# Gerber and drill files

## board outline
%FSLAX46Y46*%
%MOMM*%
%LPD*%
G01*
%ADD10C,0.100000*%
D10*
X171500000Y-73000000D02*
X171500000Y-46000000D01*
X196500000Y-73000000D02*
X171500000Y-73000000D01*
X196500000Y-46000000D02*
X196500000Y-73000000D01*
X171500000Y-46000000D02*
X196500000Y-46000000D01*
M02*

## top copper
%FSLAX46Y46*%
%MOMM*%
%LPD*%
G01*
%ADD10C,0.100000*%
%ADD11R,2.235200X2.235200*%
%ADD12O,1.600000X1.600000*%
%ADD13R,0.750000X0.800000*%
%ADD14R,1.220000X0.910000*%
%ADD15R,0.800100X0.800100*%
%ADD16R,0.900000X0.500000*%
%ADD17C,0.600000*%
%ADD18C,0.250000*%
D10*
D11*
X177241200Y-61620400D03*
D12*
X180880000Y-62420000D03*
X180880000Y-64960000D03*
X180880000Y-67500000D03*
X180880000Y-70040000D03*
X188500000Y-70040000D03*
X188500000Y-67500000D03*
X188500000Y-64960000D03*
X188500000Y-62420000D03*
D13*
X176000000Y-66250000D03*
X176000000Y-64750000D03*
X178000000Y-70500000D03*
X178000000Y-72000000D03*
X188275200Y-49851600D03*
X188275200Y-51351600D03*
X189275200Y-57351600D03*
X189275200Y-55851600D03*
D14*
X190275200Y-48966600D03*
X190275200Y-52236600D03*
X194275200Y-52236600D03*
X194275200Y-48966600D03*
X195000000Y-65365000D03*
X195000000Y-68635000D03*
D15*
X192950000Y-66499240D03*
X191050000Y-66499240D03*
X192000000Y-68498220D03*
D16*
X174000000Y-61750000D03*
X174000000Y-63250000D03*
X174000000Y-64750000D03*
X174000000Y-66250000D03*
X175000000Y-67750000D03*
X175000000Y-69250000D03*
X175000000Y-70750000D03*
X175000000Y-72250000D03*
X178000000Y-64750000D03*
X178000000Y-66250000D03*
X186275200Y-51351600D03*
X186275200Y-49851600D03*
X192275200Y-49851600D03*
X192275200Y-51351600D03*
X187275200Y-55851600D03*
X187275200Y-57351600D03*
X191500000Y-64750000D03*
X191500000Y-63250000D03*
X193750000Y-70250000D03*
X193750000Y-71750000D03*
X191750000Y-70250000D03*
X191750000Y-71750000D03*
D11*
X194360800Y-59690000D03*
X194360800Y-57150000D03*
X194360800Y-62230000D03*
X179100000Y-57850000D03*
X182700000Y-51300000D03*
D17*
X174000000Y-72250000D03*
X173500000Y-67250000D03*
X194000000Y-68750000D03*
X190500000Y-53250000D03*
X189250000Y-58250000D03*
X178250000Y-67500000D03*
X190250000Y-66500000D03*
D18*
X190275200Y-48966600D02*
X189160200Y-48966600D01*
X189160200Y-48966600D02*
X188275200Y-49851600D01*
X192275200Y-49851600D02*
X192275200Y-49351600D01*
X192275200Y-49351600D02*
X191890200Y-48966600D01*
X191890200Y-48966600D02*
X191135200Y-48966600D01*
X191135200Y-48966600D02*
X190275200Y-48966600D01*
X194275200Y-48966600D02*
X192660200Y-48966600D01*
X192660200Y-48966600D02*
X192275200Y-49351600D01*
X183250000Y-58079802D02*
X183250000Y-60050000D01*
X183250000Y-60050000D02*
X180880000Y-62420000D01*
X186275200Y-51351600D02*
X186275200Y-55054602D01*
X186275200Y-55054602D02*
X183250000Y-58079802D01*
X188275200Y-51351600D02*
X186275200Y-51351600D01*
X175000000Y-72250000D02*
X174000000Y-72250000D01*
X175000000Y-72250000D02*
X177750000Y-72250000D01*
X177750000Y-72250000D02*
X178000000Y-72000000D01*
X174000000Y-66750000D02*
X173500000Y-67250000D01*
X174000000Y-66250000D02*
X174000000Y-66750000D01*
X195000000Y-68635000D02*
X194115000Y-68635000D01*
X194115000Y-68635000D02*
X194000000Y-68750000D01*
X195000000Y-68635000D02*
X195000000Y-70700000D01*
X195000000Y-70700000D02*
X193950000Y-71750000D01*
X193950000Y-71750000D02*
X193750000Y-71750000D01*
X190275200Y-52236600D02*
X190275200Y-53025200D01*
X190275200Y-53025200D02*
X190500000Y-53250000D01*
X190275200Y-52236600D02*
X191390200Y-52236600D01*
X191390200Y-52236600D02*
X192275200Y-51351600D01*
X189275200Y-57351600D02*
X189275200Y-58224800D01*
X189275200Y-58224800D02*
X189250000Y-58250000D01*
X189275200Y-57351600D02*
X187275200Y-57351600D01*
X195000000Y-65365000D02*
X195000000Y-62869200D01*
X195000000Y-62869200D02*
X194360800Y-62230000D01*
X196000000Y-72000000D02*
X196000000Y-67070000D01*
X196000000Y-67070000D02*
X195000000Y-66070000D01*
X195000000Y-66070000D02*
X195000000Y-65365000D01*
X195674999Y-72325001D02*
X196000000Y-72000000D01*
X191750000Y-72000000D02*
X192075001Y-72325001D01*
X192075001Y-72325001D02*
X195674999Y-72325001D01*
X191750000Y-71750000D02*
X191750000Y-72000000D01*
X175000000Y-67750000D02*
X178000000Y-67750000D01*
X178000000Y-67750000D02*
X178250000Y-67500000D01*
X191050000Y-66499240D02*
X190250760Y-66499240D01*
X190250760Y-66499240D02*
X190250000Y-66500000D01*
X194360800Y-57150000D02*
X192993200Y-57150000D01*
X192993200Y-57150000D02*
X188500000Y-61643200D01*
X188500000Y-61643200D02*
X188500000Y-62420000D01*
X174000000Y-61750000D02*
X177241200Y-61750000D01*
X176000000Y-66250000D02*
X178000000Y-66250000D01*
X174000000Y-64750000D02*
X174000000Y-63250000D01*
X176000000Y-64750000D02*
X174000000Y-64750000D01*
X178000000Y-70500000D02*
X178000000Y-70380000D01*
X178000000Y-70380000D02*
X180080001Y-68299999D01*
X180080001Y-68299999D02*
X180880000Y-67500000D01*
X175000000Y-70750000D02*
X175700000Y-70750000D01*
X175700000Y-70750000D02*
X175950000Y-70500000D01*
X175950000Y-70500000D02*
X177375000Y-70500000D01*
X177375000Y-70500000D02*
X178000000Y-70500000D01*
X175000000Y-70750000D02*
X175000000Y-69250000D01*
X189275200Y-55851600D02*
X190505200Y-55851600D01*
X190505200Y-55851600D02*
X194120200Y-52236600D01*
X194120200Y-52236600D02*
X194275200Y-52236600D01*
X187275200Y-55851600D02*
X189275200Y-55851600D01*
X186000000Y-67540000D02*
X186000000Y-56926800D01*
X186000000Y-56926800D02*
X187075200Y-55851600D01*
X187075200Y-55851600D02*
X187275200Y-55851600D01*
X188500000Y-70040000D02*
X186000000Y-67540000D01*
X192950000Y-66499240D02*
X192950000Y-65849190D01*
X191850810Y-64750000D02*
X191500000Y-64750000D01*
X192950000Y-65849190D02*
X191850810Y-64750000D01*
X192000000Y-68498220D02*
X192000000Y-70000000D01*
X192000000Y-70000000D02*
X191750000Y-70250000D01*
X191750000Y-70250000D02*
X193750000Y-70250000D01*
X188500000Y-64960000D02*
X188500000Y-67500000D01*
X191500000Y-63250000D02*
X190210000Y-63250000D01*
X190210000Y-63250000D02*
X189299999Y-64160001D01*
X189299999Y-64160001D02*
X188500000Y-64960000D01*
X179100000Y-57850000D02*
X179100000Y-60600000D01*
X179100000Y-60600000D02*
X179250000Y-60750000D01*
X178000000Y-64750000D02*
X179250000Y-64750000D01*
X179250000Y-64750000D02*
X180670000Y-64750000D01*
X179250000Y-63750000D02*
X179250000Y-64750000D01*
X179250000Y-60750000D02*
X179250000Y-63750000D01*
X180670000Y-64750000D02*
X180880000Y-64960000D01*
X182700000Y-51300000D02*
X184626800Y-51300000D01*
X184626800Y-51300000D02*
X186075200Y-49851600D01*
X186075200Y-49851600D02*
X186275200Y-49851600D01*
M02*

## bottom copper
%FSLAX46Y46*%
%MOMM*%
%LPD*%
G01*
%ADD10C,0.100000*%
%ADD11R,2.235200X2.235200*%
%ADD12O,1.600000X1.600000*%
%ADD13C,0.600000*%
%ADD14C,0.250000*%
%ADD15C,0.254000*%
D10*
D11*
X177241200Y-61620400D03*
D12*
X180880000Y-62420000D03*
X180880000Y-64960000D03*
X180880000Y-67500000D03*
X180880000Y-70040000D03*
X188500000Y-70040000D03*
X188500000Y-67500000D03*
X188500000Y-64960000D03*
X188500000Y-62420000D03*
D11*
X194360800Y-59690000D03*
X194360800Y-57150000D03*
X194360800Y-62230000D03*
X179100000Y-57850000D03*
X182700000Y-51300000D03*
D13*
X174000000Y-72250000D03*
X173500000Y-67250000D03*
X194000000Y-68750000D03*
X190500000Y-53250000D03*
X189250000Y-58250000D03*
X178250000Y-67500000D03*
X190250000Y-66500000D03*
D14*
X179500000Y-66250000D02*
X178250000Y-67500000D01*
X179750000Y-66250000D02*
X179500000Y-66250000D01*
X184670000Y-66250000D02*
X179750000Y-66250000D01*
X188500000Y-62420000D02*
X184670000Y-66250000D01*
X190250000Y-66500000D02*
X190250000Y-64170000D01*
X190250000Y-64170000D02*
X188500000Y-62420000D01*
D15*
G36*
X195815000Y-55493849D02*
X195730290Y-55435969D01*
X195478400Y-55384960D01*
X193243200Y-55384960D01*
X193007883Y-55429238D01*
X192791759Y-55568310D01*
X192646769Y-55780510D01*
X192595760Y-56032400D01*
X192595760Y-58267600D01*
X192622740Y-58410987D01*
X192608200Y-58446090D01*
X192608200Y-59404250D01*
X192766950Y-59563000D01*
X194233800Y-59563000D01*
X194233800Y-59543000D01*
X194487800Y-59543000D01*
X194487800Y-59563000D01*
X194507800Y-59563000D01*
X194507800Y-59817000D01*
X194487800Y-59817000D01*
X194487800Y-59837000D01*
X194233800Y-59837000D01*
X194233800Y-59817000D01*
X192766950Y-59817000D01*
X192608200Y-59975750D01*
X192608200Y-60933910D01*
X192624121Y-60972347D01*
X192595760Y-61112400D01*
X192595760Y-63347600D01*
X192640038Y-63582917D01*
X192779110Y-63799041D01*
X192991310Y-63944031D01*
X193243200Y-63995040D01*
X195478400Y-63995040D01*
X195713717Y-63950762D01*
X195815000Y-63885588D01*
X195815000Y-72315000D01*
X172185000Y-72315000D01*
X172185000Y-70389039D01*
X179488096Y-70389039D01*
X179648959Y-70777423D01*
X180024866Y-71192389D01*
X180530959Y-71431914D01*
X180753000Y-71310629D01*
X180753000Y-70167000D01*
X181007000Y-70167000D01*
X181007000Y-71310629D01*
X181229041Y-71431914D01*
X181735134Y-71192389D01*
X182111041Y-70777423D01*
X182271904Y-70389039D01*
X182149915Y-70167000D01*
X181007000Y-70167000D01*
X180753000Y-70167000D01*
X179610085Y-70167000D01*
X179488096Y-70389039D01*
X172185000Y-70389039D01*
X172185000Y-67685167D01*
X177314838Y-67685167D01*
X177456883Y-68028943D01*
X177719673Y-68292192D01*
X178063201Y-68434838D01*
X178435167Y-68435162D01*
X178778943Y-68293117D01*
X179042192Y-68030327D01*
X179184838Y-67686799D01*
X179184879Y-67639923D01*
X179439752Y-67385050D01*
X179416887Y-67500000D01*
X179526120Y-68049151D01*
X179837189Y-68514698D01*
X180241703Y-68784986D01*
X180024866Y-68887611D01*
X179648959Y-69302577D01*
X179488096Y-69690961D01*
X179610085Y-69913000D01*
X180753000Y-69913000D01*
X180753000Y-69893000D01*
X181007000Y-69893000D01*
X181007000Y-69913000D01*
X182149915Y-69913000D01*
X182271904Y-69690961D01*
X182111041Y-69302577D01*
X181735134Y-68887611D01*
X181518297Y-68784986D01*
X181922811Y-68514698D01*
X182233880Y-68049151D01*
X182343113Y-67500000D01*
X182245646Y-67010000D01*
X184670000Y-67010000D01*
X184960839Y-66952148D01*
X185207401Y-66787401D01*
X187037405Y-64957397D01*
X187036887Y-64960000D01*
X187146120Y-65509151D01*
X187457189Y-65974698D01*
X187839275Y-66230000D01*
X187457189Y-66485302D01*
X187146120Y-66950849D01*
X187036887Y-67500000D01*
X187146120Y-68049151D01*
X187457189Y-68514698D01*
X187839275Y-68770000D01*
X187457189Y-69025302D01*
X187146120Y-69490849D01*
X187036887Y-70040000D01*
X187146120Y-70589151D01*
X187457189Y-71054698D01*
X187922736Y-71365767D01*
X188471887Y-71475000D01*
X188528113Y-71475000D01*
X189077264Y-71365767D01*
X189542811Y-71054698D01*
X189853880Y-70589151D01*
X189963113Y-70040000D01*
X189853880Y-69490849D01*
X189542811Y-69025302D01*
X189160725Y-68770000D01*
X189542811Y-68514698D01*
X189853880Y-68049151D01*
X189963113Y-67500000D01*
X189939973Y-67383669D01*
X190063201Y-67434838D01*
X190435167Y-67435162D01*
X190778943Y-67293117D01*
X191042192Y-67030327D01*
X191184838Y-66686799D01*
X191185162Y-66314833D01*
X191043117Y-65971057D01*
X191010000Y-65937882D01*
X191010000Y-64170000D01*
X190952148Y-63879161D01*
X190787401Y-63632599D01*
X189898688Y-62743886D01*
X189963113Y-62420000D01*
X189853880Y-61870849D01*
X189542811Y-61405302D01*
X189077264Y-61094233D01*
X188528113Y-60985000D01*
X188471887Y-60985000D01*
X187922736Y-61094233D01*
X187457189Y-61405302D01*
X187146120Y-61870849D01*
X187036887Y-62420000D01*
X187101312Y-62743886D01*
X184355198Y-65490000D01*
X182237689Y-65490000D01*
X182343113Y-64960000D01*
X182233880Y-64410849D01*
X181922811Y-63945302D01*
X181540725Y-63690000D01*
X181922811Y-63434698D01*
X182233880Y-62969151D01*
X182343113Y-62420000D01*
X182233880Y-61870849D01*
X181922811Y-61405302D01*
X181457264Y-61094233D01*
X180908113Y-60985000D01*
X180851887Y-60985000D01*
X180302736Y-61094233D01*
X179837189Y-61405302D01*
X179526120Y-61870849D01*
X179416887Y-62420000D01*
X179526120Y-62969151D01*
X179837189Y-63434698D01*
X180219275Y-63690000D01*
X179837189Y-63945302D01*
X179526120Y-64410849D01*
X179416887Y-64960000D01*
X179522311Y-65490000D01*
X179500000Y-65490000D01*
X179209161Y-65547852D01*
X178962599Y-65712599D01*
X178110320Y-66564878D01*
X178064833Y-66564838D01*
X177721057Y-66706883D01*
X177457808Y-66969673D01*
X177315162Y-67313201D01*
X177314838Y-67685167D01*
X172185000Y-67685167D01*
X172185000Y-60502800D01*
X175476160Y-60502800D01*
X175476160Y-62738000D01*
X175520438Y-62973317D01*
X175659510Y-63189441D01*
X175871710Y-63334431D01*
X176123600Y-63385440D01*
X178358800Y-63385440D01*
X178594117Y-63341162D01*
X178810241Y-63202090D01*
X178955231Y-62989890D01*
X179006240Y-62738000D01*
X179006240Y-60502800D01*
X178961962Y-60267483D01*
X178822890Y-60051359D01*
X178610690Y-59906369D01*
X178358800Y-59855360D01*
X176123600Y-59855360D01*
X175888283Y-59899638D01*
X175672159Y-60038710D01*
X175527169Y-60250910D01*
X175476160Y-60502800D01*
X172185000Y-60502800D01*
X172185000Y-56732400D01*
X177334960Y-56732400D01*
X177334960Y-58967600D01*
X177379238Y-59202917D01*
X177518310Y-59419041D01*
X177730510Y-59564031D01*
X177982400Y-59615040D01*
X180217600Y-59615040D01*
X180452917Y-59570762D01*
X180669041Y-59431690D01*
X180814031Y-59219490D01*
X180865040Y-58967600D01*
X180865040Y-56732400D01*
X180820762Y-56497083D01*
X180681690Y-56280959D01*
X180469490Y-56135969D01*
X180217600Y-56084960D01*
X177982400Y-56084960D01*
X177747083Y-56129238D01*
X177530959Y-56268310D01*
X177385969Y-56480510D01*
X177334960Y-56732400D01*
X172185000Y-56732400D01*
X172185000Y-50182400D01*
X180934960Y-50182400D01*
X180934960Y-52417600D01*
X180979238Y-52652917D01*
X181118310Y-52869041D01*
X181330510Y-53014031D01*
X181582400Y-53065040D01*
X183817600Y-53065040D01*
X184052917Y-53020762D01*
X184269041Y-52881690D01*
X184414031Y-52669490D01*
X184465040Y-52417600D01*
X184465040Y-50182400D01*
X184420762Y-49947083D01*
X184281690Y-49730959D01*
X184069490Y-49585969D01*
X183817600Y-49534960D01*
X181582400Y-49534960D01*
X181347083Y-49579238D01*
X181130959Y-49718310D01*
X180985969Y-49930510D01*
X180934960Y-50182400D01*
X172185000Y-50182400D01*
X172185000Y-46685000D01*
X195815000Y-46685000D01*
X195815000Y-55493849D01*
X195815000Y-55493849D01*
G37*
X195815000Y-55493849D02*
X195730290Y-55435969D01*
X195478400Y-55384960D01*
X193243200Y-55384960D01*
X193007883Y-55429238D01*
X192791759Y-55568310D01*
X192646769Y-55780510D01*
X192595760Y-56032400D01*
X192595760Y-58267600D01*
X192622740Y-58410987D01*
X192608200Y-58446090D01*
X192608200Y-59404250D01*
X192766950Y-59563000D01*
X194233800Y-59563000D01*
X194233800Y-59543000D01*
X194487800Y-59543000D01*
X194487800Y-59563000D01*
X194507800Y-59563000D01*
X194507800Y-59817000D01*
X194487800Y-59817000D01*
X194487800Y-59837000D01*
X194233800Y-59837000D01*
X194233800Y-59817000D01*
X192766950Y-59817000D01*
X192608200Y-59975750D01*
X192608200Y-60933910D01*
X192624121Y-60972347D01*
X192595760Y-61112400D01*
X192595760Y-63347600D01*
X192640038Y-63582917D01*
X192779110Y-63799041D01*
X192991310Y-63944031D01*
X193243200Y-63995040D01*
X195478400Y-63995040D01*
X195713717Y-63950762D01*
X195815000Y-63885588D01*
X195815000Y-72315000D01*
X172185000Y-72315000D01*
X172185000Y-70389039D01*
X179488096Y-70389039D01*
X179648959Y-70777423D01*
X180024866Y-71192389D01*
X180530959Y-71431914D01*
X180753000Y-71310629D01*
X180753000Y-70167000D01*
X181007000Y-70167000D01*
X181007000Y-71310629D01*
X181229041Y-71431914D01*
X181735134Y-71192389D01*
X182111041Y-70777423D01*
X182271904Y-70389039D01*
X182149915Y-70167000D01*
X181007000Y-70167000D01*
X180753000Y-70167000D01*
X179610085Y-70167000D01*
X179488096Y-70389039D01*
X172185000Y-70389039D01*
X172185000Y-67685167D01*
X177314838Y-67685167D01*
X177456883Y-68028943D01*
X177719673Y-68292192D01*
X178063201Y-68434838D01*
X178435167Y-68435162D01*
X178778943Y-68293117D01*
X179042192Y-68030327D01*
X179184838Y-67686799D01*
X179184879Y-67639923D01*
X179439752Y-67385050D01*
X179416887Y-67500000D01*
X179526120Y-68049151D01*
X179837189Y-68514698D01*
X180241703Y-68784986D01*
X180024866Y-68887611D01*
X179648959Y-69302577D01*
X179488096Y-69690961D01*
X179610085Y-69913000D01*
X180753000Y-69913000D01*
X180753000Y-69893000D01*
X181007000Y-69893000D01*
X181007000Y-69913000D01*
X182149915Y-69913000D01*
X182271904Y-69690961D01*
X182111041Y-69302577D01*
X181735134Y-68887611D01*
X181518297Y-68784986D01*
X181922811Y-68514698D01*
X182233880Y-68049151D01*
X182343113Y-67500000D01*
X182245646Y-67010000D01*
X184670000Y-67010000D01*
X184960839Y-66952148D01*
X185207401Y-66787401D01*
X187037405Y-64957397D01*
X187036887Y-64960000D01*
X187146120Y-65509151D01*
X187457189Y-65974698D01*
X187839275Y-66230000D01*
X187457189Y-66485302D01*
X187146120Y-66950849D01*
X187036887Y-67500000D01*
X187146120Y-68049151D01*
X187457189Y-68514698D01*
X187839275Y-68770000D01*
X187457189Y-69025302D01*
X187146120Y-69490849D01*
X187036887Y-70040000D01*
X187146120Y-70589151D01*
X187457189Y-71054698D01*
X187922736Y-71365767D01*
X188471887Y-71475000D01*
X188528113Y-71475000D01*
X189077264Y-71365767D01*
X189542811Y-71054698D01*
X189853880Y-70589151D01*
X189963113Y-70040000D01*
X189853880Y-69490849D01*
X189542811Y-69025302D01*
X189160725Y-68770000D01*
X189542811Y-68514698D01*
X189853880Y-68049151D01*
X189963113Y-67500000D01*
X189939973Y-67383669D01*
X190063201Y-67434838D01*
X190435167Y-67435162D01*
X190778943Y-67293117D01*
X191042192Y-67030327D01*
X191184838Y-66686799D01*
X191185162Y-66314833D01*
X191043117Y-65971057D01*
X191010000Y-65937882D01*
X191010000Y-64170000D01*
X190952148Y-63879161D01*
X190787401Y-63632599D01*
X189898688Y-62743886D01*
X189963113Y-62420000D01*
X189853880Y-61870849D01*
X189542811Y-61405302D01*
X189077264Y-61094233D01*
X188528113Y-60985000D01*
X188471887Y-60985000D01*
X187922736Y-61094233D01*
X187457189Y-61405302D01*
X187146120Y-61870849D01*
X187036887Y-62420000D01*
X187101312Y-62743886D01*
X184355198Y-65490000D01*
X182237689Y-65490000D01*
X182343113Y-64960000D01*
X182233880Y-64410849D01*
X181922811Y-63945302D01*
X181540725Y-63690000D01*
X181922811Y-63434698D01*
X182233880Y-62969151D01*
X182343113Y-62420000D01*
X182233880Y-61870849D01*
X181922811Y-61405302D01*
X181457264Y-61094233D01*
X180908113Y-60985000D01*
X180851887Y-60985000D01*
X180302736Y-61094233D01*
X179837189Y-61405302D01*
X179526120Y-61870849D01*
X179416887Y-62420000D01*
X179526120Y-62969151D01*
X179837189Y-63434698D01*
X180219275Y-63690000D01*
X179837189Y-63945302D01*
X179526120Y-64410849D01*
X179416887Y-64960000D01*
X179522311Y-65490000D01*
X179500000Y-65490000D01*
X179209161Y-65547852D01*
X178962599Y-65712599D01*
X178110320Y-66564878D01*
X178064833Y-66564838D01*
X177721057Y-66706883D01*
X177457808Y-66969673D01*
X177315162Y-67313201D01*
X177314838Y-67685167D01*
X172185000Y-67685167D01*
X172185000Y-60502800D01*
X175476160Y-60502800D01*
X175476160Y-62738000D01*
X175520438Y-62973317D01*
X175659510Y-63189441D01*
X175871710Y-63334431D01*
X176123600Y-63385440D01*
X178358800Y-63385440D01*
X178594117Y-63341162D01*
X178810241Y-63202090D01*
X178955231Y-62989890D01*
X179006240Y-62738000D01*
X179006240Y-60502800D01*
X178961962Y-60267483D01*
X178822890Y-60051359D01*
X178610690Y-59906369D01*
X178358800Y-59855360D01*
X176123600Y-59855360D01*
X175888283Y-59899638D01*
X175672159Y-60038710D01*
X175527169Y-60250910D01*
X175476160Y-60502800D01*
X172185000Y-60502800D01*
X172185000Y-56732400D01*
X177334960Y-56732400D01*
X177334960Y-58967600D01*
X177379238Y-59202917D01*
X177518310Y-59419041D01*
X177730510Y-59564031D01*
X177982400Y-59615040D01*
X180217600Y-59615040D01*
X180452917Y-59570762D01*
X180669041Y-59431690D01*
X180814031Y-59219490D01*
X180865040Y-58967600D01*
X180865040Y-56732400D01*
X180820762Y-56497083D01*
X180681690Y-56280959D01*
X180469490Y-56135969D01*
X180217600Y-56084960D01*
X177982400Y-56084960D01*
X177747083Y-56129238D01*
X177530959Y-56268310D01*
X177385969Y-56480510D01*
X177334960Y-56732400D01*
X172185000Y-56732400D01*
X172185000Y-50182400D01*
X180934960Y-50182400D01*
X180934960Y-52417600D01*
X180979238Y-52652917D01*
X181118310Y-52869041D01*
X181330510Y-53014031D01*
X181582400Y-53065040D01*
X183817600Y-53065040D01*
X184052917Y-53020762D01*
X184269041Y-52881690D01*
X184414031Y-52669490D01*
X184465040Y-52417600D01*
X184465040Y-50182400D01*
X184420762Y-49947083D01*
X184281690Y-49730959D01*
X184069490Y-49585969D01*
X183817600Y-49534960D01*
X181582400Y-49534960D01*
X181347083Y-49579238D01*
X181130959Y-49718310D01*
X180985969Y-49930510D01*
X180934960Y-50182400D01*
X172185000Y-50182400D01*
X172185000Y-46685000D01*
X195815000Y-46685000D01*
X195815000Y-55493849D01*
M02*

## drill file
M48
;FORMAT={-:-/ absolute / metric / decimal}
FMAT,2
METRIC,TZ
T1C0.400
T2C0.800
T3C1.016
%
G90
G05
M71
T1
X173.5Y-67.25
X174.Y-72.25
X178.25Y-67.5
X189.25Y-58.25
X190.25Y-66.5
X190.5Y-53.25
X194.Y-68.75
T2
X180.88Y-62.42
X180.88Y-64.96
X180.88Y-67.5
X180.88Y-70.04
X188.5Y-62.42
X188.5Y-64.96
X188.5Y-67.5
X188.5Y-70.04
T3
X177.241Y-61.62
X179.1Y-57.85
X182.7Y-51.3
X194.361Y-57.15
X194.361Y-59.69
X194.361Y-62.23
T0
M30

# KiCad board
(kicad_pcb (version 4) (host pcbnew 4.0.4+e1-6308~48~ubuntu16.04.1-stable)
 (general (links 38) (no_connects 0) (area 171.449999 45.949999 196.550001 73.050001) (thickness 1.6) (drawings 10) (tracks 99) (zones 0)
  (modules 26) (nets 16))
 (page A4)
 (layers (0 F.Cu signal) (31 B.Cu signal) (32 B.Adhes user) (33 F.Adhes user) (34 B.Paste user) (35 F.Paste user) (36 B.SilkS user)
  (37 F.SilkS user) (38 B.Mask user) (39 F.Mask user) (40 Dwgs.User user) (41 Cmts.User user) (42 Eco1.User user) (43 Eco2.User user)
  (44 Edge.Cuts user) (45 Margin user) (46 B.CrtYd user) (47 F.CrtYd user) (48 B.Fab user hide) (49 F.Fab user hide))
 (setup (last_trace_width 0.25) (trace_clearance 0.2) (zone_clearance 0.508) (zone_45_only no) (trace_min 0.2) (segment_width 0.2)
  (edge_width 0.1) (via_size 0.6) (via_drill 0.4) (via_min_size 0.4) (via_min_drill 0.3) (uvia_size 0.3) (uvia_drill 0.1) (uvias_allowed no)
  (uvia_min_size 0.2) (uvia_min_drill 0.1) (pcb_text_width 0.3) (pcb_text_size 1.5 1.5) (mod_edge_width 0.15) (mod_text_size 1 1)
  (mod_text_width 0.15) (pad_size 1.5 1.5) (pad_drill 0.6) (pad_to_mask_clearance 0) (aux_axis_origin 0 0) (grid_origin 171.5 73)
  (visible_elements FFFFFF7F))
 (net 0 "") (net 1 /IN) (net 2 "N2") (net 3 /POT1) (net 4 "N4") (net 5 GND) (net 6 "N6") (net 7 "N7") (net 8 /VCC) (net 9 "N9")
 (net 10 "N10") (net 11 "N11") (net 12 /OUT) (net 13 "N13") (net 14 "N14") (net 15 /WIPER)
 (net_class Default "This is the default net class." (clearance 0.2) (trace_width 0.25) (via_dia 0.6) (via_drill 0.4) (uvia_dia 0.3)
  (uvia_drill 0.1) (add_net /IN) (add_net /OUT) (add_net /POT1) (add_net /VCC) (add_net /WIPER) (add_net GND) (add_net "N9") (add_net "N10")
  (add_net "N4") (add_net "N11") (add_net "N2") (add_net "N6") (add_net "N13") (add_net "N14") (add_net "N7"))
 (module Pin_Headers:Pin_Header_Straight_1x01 (layer F.Cu) (at 177.2412 61.6204)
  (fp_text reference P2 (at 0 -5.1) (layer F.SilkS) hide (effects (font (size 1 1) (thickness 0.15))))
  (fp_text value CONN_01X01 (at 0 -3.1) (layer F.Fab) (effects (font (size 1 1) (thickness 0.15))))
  (pad 1 thru_hole rect (at 0 0) (size 2.2352 2.2352) (drill 1.016) (layers *.Cu *.Mask F.SilkS) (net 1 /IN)))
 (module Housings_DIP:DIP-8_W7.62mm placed (layer F.Cu) (at 180.88 62.42)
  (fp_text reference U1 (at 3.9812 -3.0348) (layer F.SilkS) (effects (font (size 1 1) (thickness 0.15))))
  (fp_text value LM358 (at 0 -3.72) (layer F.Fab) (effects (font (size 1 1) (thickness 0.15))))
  (pad 1 thru_hole oval (at 0 0) (size 1.6 1.6) (drill 0.8) (layers *.Cu *.Mask F.SilkS) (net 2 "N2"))
  (pad 2 thru_hole oval (at 0 2.54) (size 1.6 1.6) (drill 0.8) (layers *.Cu *.Mask F.SilkS) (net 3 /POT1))
  (pad 3 thru_hole oval (at 0 5.08) (size 1.6 1.6) (drill 0.8) (layers *.Cu *.Mask F.SilkS) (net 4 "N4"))
  (pad 4 thru_hole oval (at 0 7.62) (size 1.6 1.6) (drill 0.8) (layers *.Cu *.Mask F.SilkS) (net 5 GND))
  (pad 5 thru_hole oval (at 7.62 7.62) (size 1.6 1.6) (drill 0.8) (layers *.Cu *.Mask F.SilkS) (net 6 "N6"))
  (pad 6 thru_hole oval (at 7.62 5.08) (size 1.6 1.6) (drill 0.8) (layers *.Cu *.Mask F.SilkS) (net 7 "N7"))
  (pad 7 thru_hole oval (at 7.62 2.54) (size 1.6 1.6) (drill 0.8) (layers *.Cu *.Mask F.SilkS) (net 7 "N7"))
  (pad 8 thru_hole oval (at 7.62 0) (size 1.6 1.6) (drill 0.8) (layers *.Cu *.Mask F.SilkS) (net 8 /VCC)))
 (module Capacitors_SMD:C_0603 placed (layer F.Cu) (at 176 65.5 90)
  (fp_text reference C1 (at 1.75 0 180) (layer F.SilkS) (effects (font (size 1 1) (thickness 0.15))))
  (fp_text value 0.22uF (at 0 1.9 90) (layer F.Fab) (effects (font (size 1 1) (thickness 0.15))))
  (pad 1 smd rect (at -0.75 0 90) (size 0.8 0.75) (layers F.Cu F.Paste F.Mask) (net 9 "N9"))
  (pad 2 smd rect (at 0.75 0 90) (size 0.8 0.75) (layers F.Cu F.Paste F.Mask) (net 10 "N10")))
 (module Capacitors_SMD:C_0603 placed (layer F.Cu) (at 178 71.25 270)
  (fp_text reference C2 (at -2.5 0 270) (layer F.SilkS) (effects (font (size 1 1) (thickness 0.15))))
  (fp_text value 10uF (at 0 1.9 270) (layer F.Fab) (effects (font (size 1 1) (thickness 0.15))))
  (pad 1 smd rect (at -0.75 0 270) (size 0.8 0.75) (layers F.Cu F.Paste F.Mask) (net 4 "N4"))
  (pad 2 smd rect (at 0.75 0 270) (size 0.8 0.75) (layers F.Cu F.Paste F.Mask) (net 5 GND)))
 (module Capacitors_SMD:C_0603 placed (layer F.Cu) (at 188.2752 50.6016 270)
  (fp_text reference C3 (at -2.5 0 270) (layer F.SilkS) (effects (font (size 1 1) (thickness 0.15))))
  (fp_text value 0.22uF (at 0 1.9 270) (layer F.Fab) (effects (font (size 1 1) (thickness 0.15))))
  (pad 1 smd rect (at -0.75 0 270) (size 0.8 0.75) (layers F.Cu F.Paste F.Mask) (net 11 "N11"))
  (pad 2 smd rect (at 0.75 0 270) (size 0.8 0.75) (layers F.Cu F.Paste F.Mask) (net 2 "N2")))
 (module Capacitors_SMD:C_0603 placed (layer F.Cu) (at 189.2752 56.6016 90)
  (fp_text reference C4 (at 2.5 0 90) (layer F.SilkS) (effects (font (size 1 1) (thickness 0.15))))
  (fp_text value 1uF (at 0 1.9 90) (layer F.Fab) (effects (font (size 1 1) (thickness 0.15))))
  (pad 1 smd rect (at -0.75 0 90) (size 0.8 0.75) (layers F.Cu F.Paste F.Mask) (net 5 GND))
  (pad 2 smd rect (at 0.75 0 90) (size 0.8 0.75) (layers F.Cu F.Paste F.Mask) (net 6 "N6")))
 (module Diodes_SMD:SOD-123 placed (layer F.Cu) (at 190.2752 50.6016 270)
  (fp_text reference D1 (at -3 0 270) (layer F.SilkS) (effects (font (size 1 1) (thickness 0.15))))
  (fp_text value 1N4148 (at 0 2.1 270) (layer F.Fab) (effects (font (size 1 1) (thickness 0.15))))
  (pad 1 smd rect (at -1.635 0 270) (size 0.91 1.22) (layers F.Cu F.Paste F.Mask) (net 11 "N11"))
  (pad 2 smd rect (at 1.635 0 270) (size 0.91 1.22) (layers F.Cu F.Paste F.Mask) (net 5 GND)))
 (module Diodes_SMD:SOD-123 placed (layer F.Cu) (at 194.2752 50.6016 90)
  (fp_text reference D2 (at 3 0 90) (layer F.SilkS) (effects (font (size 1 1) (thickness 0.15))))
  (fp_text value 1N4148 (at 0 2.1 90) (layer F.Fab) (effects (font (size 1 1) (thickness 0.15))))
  (pad 1 smd rect (at -1.635 0 90) (size 0.91 1.22) (layers F.Cu F.Paste F.Mask) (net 6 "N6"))
  (pad 2 smd rect (at 1.635 0 90) (size 0.91 1.22) (layers F.Cu F.Paste F.Mask) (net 11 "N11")))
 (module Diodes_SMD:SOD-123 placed (layer F.Cu) (at 195 67 270)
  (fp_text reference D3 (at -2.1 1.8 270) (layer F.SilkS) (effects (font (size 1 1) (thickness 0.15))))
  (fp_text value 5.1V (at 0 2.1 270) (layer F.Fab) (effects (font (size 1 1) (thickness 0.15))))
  (pad 1 smd rect (at -1.635 0 270) (size 0.91 1.22) (layers F.Cu F.Paste F.Mask) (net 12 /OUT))
  (pad 2 smd rect (at 1.635 0 270) (size 0.91 1.22) (layers F.Cu F.Paste F.Mask) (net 5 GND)))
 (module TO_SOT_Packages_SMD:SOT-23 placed (layer F.Cu) (at 192 67.5 180)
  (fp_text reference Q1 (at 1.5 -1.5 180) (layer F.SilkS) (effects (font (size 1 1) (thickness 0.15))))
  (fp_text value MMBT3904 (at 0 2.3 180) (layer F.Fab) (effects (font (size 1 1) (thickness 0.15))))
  (pad 1 smd rect (at -0.95 1.00076 180) (size 0.8001 0.8001) (layers F.Cu F.Paste F.Mask) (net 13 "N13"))
  (pad 2 smd rect (at 0.95 1.00076 180) (size 0.8001 0.8001) (layers F.Cu F.Paste F.Mask) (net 8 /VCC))
  (pad 3 smd rect (at 0 -0.99822 180) (size 0.8001 0.8001) (layers F.Cu F.Paste F.Mask) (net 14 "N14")))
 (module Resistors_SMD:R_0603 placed (layer F.Cu) (at 174 62.5 270)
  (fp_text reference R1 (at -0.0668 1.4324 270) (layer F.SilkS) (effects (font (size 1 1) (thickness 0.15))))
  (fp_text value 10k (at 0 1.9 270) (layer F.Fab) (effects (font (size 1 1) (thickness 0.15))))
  (pad 1 smd rect (at -0.75 0 270) (size 0.5 0.9) (layers F.Cu F.Paste F.Mask) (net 1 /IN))
  (pad 2 smd rect (at 0.75 0 270) (size 0.5 0.9) (layers F.Cu F.Paste F.Mask) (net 10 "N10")))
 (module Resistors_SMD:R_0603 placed (layer F.Cu) (at 174 65.5 270)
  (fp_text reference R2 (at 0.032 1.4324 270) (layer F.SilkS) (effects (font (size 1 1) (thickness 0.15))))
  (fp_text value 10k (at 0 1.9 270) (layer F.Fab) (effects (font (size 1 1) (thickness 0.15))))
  (pad 1 smd rect (at -0.75 0 270) (size 0.5 0.9) (layers F.Cu F.Paste F.Mask) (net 10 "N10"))
  (pad 2 smd rect (at 0.75 0 270) (size 0.5 0.9) (layers F.Cu F.Paste F.Mask) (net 5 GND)))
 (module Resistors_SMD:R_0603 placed (layer F.Cu) (at 175 68.5 270)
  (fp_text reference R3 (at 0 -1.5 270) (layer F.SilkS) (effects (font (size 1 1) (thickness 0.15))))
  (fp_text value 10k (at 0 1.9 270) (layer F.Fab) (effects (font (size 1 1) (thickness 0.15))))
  (pad 1 smd rect (at -0.75 0 270) (size 0.5 0.9) (layers F.Cu F.Paste F.Mask) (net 8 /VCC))
  (pad 2 smd rect (at 0.75 0 270) (size 0.5 0.9) (layers F.Cu F.Paste F.Mask) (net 4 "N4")))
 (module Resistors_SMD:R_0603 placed (layer F.Cu) (at 175 71.5 270)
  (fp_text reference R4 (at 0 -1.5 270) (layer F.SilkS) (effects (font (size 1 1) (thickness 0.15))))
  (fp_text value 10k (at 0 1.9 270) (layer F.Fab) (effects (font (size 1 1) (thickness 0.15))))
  (pad 1 smd rect (at -0.75 0 270) (size 0.5 0.9) (layers F.Cu F.Paste F.Mask) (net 4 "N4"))
  (pad 2 smd rect (at 0.75 0 270) (size 0.5 0.9) (layers F.Cu F.Paste F.Mask) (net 5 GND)))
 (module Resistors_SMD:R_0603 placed (layer F.Cu) (at 178 65.5 270)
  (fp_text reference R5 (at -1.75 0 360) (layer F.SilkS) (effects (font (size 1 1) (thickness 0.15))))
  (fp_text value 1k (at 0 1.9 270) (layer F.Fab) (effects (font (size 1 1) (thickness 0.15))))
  (pad 1 smd rect (at -0.75 0 270) (size 0.5 0.9) (layers F.Cu F.Paste F.Mask) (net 3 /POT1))
  (pad 2 smd rect (at 0.75 0 270) (size 0.5 0.9) (layers F.Cu F.Paste F.Mask) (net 9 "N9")))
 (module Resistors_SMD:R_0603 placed (layer F.Cu) (at 186.2752 50.6016 90)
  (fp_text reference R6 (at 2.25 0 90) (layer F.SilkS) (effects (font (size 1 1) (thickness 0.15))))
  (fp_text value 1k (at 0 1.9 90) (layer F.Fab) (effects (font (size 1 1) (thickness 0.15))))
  (pad 1 smd rect (at -0.75 0 90) (size 0.5 0.9) (layers F.Cu F.Paste F.Mask) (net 2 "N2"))
  (pad 2 smd rect (at 0.75 0 90) (size 0.5 0.9) (layers F.Cu F.Paste F.Mask) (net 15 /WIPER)))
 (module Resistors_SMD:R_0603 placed (layer F.Cu) (at 192.2752 50.6016 270)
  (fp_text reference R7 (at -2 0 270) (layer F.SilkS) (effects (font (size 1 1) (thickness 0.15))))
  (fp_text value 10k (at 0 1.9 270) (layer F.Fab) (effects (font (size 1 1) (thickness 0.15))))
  (pad 1 smd rect (at -0.75 0 270) (size 0.5 0.9) (layers F.Cu F.Paste F.Mask) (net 11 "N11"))
  (pad 2 smd rect (at 0.75 0 270) (size 0.5 0.9) (layers F.Cu F.Paste F.Mask) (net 5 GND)))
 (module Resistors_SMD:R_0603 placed (layer F.Cu) (at 187.2752 56.6016 270)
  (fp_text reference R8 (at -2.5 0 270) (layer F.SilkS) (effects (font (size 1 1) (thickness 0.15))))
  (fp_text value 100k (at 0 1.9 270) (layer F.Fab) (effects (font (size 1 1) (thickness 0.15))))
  (pad 1 smd rect (at -0.75 0 270) (size 0.5 0.9) (layers F.Cu F.Paste F.Mask) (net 6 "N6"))
  (pad 2 smd rect (at 0.75 0 270) (size 0.5 0.9) (layers F.Cu F.Paste F.Mask) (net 5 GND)))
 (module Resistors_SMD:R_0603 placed (layer F.Cu) (at 191.5 64 90)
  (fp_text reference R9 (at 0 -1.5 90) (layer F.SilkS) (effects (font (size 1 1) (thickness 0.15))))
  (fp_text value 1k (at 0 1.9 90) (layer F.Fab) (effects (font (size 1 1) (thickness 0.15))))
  (pad 1 smd rect (at -0.75 0 90) (size 0.5 0.9) (layers F.Cu F.Paste F.Mask) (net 13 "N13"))
  (pad 2 smd rect (at 0.75 0 90) (size 0.5 0.9) (layers F.Cu F.Paste F.Mask) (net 7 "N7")))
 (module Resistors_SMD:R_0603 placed (layer F.Cu) (at 193.75 71 270)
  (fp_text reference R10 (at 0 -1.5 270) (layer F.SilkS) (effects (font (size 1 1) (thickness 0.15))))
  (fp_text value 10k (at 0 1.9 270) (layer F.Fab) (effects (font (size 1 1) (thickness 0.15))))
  (pad 1 smd rect (at -0.75 0 270) (size 0.5 0.9) (layers F.Cu F.Paste F.Mask) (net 14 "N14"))
  (pad 2 smd rect (at 0.75 0 270) (size 0.5 0.9) (layers F.Cu F.Paste F.Mask) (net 5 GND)))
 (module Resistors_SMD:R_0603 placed (layer F.Cu) (at 191.75 71 270)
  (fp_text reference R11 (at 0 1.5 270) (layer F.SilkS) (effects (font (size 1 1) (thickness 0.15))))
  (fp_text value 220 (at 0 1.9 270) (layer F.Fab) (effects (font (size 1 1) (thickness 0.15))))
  (pad 1 smd rect (at -0.75 0 270) (size 0.5 0.9) (layers F.Cu F.Paste F.Mask) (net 14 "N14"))
  (pad 2 smd rect (at 0.75 0 270) (size 0.5 0.9) (layers F.Cu F.Paste F.Mask) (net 12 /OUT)))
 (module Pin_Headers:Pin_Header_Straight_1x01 (layer F.Cu) (at 194.3608 59.69)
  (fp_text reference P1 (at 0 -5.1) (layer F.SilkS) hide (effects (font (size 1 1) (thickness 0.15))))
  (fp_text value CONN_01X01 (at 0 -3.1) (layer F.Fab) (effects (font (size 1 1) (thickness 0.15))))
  (pad 1 thru_hole rect (at 0 0) (size 2.2352 2.2352) (drill 1.016) (layers *.Cu *.Mask F.SilkS) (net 5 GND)))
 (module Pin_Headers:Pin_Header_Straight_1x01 (layer F.Cu) (at 194.3608 57.15)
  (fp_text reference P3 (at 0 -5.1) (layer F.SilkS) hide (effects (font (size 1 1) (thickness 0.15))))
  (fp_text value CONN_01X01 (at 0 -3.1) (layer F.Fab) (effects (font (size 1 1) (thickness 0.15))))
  (pad 1 thru_hole rect (at 0 0) (size 2.2352 2.2352) (drill 1.016) (layers *.Cu *.Mask F.SilkS) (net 8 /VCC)))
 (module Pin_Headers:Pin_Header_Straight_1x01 (layer F.Cu) (at 194.3608 62.23)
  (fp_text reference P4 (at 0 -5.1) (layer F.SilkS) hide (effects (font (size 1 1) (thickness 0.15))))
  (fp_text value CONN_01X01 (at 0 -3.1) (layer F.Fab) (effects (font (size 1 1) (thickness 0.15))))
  (pad 1 thru_hole rect (at 0 0) (size 2.2352 2.2352) (drill 1.016) (layers *.Cu *.Mask F.SilkS) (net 12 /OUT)))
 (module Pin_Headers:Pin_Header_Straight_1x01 (layer F.Cu) (at 179.1 57.85)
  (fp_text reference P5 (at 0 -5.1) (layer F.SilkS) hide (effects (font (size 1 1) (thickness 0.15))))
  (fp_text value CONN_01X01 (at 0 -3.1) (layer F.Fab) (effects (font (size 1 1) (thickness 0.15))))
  (pad 1 thru_hole rect (at 0 0) (size 2.2352 2.2352) (drill 1.016) (layers *.Cu *.Mask F.SilkS) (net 3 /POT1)))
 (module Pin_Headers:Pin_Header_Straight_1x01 (layer F.Cu) (at 182.7 51.3)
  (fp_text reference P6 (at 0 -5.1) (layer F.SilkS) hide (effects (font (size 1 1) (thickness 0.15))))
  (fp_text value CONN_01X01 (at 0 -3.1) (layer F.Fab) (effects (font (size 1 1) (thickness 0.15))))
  (pad 1 thru_hole rect (at 0 0) (size 2.2352 2.2352) (drill 1.016) (layers *.Cu *.Mask F.SilkS) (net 15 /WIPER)))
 (gr_line (start 171.5 73) (end 171.5 46) (layer Edge.Cuts) (width 0.1))
 (gr_line (start 196.5 73) (end 171.5 73) (layer Edge.Cuts) (width 0.1))
 (gr_line (start 196.5 46) (end 196.5 73) (layer Edge.Cuts) (width 0.1))
 (gr_line (start 171.5 46) (end 196.5 46) (layer Edge.Cuts) (width 0.1))
 (segment (start 190.2752 48.9666) (end 189.1602 48.9666) (width 0.25) (layer F.Cu) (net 11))
 (segment (start 189.1602 48.9666) (end 188.2752 49.8516) (width 0.25) (layer F.Cu) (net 11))
 (segment (start 192.2752 49.8516) (end 192.2752 49.3516) (width 0.25) (layer F.Cu) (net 11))
 (segment (start 192.2752 49.3516) (end 191.8902 48.9666) (width 0.25) (layer F.Cu) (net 11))
 (segment (start 191.8902 48.9666) (end 191.1352 48.9666) (width 0.25) (layer F.Cu) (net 11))
 (segment (start 191.1352 48.9666) (end 190.2752 48.9666) (width 0.25) (layer F.Cu) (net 11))
 (segment (start 194.2752 48.9666) (end 192.6602 48.9666) (width 0.25) (layer F.Cu) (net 11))
 (segment (start 192.6602 48.9666) (end 192.2752 49.3516) (width 0.25) (layer F.Cu) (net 11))
 (segment (start 183.25 58.079802) (end 183.25 60.05) (width 0.25) (layer F.Cu) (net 2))
 (segment (start 183.25 60.05) (end 180.88 62.42) (width 0.25) (layer F.Cu) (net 2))
 (segment (start 186.2752 51.3516) (end 186.2752 55.054602) (width 0.25) (layer F.Cu) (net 2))
 (segment (start 186.2752 55.054602) (end 183.25 58.079802) (width 0.25) (layer F.Cu) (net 2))
 (segment (start 188.2752 51.3516) (end 186.2752 51.3516) (width 0.25) (layer F.Cu) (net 2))
 (segment (start 175 72.25) (end 174 72.25) (width 0.25) (layer F.Cu) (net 5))
 (via (at 174 72.25) (size 0.6) (drill 0.4) (layers F.Cu B.Cu) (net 5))
 (segment (start 175 72.25) (end 177.75 72.25) (width 0.25) (layer F.Cu) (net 5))
 (segment (start 177.75 72.25) (end 178 72) (width 0.25) (layer F.Cu) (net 5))
 (segment (start 174 66.75) (end 173.5 67.25) (width 0.25) (layer F.Cu) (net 5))
 (via (at 173.5 67.25) (size 0.6) (drill 0.4) (layers F.Cu B.Cu) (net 5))
 (segment (start 174 66.25) (end 174 66.75) (width 0.25) (layer F.Cu) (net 5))
 (segment (start 195 68.635) (end 194.115 68.635) (width 0.25) (layer F.Cu) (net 5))
 (segment (start 194.115 68.635) (end 194 68.75) (width 0.25) (layer F.Cu) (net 5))
 (via (at 194 68.75) (size 0.6) (drill 0.4) (layers F.Cu B.Cu) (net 5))
 (segment (start 195 68.635) (end 195 70.7) (width 0.25) (layer F.Cu) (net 5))
 (segment (start 195 70.7) (end 193.95 71.75) (width 0.25) (layer F.Cu) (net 5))
 (segment (start 193.95 71.75) (end 193.75 71.75) (width 0.25) (layer F.Cu) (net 5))
 (segment (start 190.2752 52.2366) (end 190.2752 53.0252) (width 0.25) (layer F.Cu) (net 5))
 (segment (start 190.2752 53.0252) (end 190.5 53.25) (width 0.25) (layer F.Cu) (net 5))
 (via (at 190.5 53.25) (size 0.6) (drill 0.4) (layers F.Cu B.Cu) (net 5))
 (segment (start 190.2752 52.2366) (end 191.3902 52.2366) (width 0.25) (layer F.Cu) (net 5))
 (segment (start 191.3902 52.2366) (end 192.2752 51.3516) (width 0.25) (layer F.Cu) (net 5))
 (segment (start 189.2752 57.3516) (end 189.2752 58.2248) (width 0.25) (layer F.Cu) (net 5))
 (segment (start 189.2752 58.2248) (end 189.25 58.25) (width 0.25) (layer F.Cu) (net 5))
 (via (at 189.25 58.25) (size 0.6) (drill 0.4) (layers F.Cu B.Cu) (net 5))
 (segment (start 189.2752 57.3516) (end 187.2752 57.3516) (width 0.25) (layer F.Cu) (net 5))
 (segment (start 195 65.365) (end 195 62.8692) (width 0.25) (layer F.Cu) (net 12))
 (segment (start 195 62.8692) (end 194.3608 62.23) (width 0.25) (layer F.Cu) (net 12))
 (segment (start 196 72) (end 196 67.07) (width 0.25) (layer F.Cu) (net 12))
 (segment (start 196 67.07) (end 195 66.07) (width 0.25) (layer F.Cu) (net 12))
 (segment (start 195 66.07) (end 195 65.365) (width 0.25) (layer F.Cu) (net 12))
 (segment (start 195.674999 72.325001) (end 196 72) (width 0.25) (layer F.Cu) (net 12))
 (segment (start 191.75 72) (end 192.075001 72.325001) (width 0.25) (layer F.Cu) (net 12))
 (segment (start 192.075001 72.325001) (end 195.674999 72.325001) (width 0.25) (layer F.Cu) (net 12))
 (segment (start 191.75 71.75) (end 191.75 72) (width 0.25) (layer F.Cu) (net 12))
 (segment (start 175 67.75) (end 178 67.75) (width 0.25) (layer F.Cu) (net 8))
 (segment (start 178 67.75) (end 178.25 67.5) (width 0.25) (layer F.Cu) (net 8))
 (via (at 178.25 67.5) (size 0.6) (drill 0.4) (layers F.Cu B.Cu) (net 8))
 (segment (start 179.5 66.25) (end 178.25 67.5) (width 0.25) (layer B.Cu) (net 8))
 (segment (start 179.75 66.25) (end 179.5 66.25) (width 0.25) (layer B.Cu) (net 8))
 (segment (start 184.67 66.25) (end 179.75 66.25) (width 0.25) (layer B.Cu) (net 8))
 (segment (start 188.5 62.42) (end 184.67 66.25) (width 0.25) (layer B.Cu) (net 8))
 (segment (start 190.25 66.5) (end 190.25 64.17) (width 0.25) (layer B.Cu) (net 8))
 (segment (start 190.25 64.17) (end 188.5 62.42) (width 0.25) (layer B.Cu) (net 8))
 (segment (start 191.05 66.49924) (end 190.25076 66.49924) (width 0.25) (layer F.Cu) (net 8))
 (segment (start 190.25076 66.49924) (end 190.25 66.5) (width 0.25) (layer F.Cu) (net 8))
 (via (at 190.25 66.5) (size 0.6) (drill 0.4) (layers F.Cu B.Cu) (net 8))
 (segment (start 194.3608 57.15) (end 192.9932 57.15) (width 0.25) (layer F.Cu) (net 8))
 (segment (start 192.9932 57.15) (end 188.5 61.6432) (width 0.25) (layer F.Cu) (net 8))
 (segment (start 188.5 61.6432) (end 188.5 62.42) (width 0.25) (layer F.Cu) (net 8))
 (segment (start 174 61.75) (end 177.2412 61.75) (width 0.25) (layer F.Cu) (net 1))
 (segment (start 176 66.25) (end 178 66.25) (width 0.25) (layer F.Cu) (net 9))
 (segment (start 174 64.75) (end 174 63.25) (width 0.25) (layer F.Cu) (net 10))
 (segment (start 176 64.75) (end 174 64.75) (width 0.25) (layer F.Cu) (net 10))
 (segment (start 178 70.5) (end 178 70.38) (width 0.25) (layer F.Cu) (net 4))
 (segment (start 178 70.38) (end 180.080001 68.299999) (width 0.25) (layer F.Cu) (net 4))
 (segment (start 180.080001 68.299999) (end 180.88 67.5) (width 0.25) (layer F.Cu) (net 4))
 (segment (start 175 70.75) (end 175.7 70.75) (width 0.25) (layer F.Cu) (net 4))
 (segment (start 175.7 70.75) (end 175.95 70.5) (width 0.25) (layer F.Cu) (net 4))
 (segment (start 175.95 70.5) (end 177.375 70.5) (width 0.25) (layer F.Cu) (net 4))
 (segment (start 177.375 70.5) (end 178 70.5) (width 0.25) (layer F.Cu) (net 4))
 (segment (start 175 70.75) (end 175 69.25) (width 0.25) (layer F.Cu) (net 4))
 (segment (start 189.2752 55.8516) (end 190.5052 55.8516) (width 0.25) (layer F.Cu) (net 6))
 (segment (start 190.5052 55.8516) (end 194.1202 52.2366) (width 0.25) (layer F.Cu) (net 6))
 (segment (start 194.1202 52.2366) (end 194.2752 52.2366) (width 0.25) (layer F.Cu) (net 6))
 (segment (start 187.2752 55.8516) (end 189.2752 55.8516) (width 0.25) (layer F.Cu) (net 6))
 (segment (start 186 67.54) (end 186 56.9268) (width 0.25) (layer F.Cu) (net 6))
 (segment (start 186 56.9268) (end 187.0752 55.8516) (width 0.25) (layer F.Cu) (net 6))
 (segment (start 187.0752 55.8516) (end 187.2752 55.8516) (width 0.25) (layer F.Cu) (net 6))
 (segment (start 188.5 70.04) (end 186 67.54) (width 0.25) (layer F.Cu) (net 6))
 (segment (start 192.95 66.49924) (end 192.95 65.84919) (width 0.25) (layer F.Cu) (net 13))
 (segment (start 191.85081 64.75) (end 191.5 64.75) (width 0.25) (layer F.Cu) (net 13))
 (segment (start 192.95 65.84919) (end 191.85081 64.75) (width 0.25) (layer F.Cu) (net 13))
 (segment (start 192 68.49822) (end 192 70) (width 0.25) (layer F.Cu) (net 14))
 (segment (start 192 70) (end 191.75 70.25) (width 0.25) (layer F.Cu) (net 14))
 (segment (start 191.75 70.25) (end 193.75 70.25) (width 0.25) (layer F.Cu) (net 14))
 (segment (start 188.5 64.96) (end 188.5 67.5) (width 0.25) (layer F.Cu) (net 7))
 (segment (start 191.5 63.25) (end 190.21 63.25) (width 0.25) (layer F.Cu) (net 7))
 (segment (start 190.21 63.25) (end 189.299999 64.160001) (width 0.25) (layer F.Cu) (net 7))
 (segment (start 189.299999 64.160001) (end 188.5 64.96) (width 0.25) (layer F.Cu) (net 7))
 (segment (start 179.1 57.85) (end 179.1 60.6) (width 0.25) (layer F.Cu) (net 3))
 (segment (start 179.1 60.6) (end 179.25 60.75) (width 0.25) (layer F.Cu) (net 3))
 (segment (start 178 64.75) (end 179.25 64.75) (width 0.25) (layer F.Cu) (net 3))
 (segment (start 179.25 64.75) (end 180.67 64.75) (width 0.25) (layer F.Cu) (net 3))
 (segment (start 179.25 63.75) (end 179.25 64.75) (width 0.25) (layer F.Cu) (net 3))
 (segment (start 179.25 60.75) (end 179.25 63.75) (width 0.25) (layer F.Cu) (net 3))
 (segment (start 180.67 64.75) (end 180.88 64.96) (width 0.25) (layer F.Cu) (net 3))
 (segment (start 182.7 51.3) (end 184.6268 51.3) (width 0.25) (layer F.Cu) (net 15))
 (segment (start 184.6268 51.3) (end 186.0752 49.8516) (width 0.25) (layer F.Cu) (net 15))
 (segment (start 186.0752 49.8516) (end 186.2752 49.8516) (width 0.25) (layer F.Cu) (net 15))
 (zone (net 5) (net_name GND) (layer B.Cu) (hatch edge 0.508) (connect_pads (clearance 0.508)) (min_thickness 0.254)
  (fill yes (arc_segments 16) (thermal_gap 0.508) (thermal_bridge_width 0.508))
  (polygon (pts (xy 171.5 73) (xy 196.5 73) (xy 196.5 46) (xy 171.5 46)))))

